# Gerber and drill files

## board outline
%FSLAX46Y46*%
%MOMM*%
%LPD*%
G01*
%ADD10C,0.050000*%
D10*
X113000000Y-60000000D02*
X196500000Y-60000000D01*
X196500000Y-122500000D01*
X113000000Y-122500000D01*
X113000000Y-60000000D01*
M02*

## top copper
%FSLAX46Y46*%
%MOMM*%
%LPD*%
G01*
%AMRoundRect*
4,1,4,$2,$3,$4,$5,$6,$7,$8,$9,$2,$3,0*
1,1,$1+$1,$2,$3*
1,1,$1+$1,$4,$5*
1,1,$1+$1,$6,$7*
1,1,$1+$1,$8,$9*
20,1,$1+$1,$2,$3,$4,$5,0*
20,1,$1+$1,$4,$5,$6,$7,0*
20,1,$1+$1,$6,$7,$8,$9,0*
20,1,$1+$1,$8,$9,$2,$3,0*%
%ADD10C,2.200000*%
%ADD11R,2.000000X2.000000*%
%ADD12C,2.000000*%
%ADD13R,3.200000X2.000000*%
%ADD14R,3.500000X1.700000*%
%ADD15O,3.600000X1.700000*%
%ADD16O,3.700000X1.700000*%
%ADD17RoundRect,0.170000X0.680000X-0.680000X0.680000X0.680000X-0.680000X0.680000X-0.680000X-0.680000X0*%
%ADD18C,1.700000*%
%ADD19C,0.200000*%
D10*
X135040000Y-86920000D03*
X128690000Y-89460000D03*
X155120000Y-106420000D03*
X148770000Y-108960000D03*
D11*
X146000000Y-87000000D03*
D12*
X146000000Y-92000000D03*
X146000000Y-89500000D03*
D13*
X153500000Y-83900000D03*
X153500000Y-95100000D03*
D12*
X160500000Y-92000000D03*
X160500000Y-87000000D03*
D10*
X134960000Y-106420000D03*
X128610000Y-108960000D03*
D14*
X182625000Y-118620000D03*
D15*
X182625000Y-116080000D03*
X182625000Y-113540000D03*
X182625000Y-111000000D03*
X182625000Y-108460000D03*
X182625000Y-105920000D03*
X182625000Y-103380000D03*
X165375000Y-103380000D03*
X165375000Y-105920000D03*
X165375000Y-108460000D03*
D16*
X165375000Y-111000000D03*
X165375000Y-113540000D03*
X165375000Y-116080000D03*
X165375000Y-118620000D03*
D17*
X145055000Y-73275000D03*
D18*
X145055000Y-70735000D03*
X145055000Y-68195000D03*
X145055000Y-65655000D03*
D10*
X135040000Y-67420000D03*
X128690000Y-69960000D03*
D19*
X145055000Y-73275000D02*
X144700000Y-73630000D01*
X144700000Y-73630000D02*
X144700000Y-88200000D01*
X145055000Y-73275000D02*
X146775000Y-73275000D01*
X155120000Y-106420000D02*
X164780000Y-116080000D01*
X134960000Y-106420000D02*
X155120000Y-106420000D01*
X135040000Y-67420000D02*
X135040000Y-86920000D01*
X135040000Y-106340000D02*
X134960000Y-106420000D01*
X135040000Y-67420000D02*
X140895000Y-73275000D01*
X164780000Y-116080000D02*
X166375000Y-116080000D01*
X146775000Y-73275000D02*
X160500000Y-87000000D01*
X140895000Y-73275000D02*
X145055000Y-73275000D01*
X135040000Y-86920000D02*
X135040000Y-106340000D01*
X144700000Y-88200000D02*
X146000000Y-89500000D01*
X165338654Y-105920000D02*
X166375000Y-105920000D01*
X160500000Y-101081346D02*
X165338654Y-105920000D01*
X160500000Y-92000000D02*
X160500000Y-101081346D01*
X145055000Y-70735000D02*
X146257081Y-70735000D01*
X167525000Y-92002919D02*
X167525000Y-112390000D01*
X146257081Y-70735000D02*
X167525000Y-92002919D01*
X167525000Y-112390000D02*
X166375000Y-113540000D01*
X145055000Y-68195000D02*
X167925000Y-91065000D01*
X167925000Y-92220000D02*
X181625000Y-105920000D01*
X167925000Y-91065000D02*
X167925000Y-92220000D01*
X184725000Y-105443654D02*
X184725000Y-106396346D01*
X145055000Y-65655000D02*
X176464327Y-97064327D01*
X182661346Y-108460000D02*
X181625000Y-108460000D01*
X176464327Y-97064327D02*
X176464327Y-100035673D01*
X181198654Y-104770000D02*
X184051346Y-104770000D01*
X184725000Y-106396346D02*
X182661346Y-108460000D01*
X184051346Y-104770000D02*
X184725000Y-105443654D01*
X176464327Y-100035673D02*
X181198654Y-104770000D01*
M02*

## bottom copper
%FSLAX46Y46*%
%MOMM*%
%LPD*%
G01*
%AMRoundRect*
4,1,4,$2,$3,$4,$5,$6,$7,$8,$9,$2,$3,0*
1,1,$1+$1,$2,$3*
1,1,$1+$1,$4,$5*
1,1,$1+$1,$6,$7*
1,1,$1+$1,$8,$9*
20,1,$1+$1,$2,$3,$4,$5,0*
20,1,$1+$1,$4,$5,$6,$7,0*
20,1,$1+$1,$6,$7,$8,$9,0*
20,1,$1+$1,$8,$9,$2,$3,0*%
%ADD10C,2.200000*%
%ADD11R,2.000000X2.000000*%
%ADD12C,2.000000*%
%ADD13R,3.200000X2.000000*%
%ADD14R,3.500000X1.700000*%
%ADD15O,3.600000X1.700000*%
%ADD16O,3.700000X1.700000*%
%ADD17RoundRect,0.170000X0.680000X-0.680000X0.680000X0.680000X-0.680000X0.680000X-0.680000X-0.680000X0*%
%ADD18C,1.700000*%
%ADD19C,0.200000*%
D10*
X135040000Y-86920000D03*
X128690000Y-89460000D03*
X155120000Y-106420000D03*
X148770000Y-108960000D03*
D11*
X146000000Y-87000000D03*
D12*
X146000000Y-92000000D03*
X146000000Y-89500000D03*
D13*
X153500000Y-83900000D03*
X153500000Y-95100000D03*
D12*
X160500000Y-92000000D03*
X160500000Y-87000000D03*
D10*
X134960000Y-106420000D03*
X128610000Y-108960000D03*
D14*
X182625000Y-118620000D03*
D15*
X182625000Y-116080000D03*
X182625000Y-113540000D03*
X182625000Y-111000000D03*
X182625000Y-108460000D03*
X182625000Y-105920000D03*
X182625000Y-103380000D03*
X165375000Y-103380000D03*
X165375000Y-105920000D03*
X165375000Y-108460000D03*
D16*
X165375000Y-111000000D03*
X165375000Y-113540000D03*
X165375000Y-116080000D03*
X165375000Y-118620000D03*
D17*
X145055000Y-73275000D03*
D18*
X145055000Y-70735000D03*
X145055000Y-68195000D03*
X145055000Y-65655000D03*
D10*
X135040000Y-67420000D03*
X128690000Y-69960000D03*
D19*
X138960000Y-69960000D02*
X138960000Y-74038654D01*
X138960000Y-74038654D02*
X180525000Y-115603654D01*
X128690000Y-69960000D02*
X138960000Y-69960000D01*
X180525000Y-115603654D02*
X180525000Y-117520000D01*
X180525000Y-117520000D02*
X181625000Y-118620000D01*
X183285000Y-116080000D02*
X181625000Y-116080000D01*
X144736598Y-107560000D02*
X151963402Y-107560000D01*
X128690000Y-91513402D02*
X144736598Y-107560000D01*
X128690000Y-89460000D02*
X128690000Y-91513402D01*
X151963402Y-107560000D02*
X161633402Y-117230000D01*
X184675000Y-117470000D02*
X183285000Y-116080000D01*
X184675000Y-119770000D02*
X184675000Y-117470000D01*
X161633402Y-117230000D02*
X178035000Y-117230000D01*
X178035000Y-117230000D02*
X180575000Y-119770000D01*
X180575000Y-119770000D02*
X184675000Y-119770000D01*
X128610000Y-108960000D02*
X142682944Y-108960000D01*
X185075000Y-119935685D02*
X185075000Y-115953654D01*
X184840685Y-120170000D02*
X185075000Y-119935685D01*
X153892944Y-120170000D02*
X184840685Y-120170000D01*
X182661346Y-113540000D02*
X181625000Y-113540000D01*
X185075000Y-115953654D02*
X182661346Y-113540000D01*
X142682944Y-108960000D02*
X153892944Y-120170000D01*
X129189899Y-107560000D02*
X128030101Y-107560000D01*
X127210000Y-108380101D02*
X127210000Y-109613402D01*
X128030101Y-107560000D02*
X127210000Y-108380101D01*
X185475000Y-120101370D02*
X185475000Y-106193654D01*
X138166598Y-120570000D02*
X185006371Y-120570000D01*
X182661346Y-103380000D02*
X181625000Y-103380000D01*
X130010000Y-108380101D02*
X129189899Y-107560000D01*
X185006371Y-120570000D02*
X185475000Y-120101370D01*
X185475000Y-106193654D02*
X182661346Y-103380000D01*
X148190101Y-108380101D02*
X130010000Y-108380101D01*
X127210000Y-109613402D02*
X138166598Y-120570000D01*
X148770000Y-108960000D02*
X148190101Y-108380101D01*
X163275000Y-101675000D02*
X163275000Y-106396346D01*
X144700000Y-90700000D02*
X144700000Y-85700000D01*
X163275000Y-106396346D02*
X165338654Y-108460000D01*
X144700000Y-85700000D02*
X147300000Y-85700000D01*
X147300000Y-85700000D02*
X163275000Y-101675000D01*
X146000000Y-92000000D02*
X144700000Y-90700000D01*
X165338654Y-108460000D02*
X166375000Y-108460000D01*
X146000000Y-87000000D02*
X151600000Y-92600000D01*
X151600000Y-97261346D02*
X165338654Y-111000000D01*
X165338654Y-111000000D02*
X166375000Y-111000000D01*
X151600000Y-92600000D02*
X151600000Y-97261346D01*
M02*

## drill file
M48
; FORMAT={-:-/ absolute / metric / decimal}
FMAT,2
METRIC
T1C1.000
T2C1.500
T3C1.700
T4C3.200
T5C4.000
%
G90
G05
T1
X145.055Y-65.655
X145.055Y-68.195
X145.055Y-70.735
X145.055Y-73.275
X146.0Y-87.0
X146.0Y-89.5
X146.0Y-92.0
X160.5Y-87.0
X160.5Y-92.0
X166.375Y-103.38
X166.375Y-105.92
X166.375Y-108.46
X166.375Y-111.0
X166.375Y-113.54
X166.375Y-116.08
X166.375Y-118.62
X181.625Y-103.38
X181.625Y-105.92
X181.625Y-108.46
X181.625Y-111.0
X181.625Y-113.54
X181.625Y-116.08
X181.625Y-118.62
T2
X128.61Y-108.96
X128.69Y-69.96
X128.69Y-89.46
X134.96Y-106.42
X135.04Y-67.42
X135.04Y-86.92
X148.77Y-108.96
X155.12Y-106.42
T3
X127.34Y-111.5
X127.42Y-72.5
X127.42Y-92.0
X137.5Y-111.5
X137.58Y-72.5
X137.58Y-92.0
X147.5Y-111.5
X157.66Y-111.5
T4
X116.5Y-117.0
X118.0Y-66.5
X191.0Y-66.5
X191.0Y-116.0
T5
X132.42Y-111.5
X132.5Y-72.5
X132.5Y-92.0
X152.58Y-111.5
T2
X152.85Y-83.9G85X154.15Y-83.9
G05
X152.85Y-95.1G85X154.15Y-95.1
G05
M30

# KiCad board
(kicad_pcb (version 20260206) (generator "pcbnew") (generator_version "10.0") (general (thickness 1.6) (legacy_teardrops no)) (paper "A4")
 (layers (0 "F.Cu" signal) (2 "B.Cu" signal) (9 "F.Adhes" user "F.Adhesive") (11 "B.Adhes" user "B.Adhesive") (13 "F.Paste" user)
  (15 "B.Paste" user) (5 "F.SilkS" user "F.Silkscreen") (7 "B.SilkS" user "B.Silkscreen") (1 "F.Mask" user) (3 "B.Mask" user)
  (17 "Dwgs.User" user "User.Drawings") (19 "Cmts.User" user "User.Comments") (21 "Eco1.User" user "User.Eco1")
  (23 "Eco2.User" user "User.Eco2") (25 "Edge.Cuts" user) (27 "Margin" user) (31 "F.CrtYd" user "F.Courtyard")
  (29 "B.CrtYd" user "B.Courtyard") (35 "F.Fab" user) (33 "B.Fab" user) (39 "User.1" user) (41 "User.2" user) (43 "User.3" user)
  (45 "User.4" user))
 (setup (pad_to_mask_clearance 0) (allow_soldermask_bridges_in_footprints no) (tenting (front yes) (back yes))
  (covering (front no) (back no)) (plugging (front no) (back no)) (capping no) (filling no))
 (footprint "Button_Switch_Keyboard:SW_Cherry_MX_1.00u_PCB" (layer "F.Cu") (at 135.04 86.92)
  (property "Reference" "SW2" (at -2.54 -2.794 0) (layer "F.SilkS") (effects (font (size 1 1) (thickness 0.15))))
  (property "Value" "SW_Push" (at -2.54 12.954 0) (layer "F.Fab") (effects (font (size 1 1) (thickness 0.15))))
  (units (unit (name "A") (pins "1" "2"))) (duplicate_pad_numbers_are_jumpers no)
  (pad "" np_thru_hole circle (at -7.62 5.08) (size 1.7 1.7) (drill 1.7) (layers "*.Cu" "*.Mask"))
  (pad "" np_thru_hole circle (at -2.54 5.08) (size 4 4) (drill 4) (layers "*.Cu" "*.Mask"))
  (pad "" np_thru_hole circle (at 2.54 5.08) (size 1.7 1.7) (drill 1.7) (layers "*.Cu" "*.Mask"))
  (pad "1" thru_hole circle (at 0 0) (size 2.2 2.2) (drill 1.5) (layers "*.Cu" "*.Mask") (remove_unused_layers no) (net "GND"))
  (pad "2" thru_hole circle (at -6.35 2.54) (size 2.2 2.2) (drill 1.5) (layers "*.Cu" "*.Mask") (remove_unused_layers no)
   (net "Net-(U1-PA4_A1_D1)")))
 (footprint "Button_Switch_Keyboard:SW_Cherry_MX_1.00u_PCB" (layer "F.Cu") (at 155.12 106.42)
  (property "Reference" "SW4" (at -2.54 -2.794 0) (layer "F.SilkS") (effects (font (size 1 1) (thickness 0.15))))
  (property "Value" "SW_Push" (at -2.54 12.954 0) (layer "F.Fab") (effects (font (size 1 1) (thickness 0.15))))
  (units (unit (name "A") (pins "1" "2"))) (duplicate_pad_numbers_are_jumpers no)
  (pad "" np_thru_hole circle (at -7.62 5.08) (size 1.7 1.7) (drill 1.7) (layers "*.Cu" "*.Mask"))
  (pad "" np_thru_hole circle (at -2.54 5.08) (size 4 4) (drill 4) (layers "*.Cu" "*.Mask"))
  (pad "" np_thru_hole circle (at 2.54 5.08) (size 1.7 1.7) (drill 1.7) (layers "*.Cu" "*.Mask"))
  (pad "1" thru_hole circle (at 0 0) (size 2.2 2.2) (drill 1.5) (layers "*.Cu" "*.Mask") (remove_unused_layers no) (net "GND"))
  (pad "2" thru_hole circle (at -6.35 2.54) (size 2.2 2.2) (drill 1.5) (layers "*.Cu" "*.Mask") (remove_unused_layers no)
   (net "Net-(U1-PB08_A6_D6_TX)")))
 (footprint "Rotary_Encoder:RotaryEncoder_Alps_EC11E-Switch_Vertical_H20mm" (layer "F.Cu") (at 146 87)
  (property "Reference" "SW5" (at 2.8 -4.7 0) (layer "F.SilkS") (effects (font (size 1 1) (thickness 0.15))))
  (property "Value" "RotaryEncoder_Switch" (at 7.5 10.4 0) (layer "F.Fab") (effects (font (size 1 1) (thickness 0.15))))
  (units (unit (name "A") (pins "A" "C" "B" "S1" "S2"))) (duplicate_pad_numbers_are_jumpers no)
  (pad "A" thru_hole rect (at 0 0) (size 2 2) (drill 1) (layers "*.Cu" "*.Mask") (remove_unused_layers no) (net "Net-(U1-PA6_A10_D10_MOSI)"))
  (pad "B" thru_hole circle (at 0 5) (size 2 2) (drill 1) (layers "*.Cu" "*.Mask") (remove_unused_layers no) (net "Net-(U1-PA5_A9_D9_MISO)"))
  (pad "C" thru_hole circle (at 0 2.5) (size 2 2) (drill 1) (layers "*.Cu" "*.Mask") (remove_unused_layers no) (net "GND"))
  (pad "MP" thru_hole rect (at 7.5 -3.1) (size 3.2 2) (drill oval 2.8 1.5) (layers "*.Cu" "*.Mask") (remove_unused_layers no))
  (pad "MP" thru_hole rect (at 7.5 8.1) (size 3.2 2) (drill oval 2.8 1.5) (layers "*.Cu" "*.Mask") (remove_unused_layers no))
  (pad "S1" thru_hole circle (at 14.5 5) (size 2 2) (drill 1) (layers "*.Cu" "*.Mask") (remove_unused_layers no)
   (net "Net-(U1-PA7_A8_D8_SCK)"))
  (pad "S2" thru_hole circle (at 14.5 0) (size 2 2) (drill 1) (layers "*.Cu" "*.Mask") (remove_unused_layers no) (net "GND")))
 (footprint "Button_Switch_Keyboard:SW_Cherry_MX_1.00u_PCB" (layer "F.Cu") (at 134.96 106.42)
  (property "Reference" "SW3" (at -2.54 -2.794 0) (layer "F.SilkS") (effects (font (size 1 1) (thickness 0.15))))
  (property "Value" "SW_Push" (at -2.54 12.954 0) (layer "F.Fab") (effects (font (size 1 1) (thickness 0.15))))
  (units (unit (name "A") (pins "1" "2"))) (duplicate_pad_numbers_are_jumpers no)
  (pad "" np_thru_hole circle (at -7.62 5.08) (size 1.7 1.7) (drill 1.7) (layers "*.Cu" "*.Mask"))
  (pad "" np_thru_hole circle (at -2.54 5.08) (size 4 4) (drill 4) (layers "*.Cu" "*.Mask"))
  (pad "" np_thru_hole circle (at 2.54 5.08) (size 1.7 1.7) (drill 1.7) (layers "*.Cu" "*.Mask"))
  (pad "1" thru_hole circle (at 0 0) (size 2.2 2.2) (drill 1.5) (layers "*.Cu" "*.Mask") (remove_unused_layers no) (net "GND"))
  (pad "2" thru_hole circle (at -6.35 2.54) (size 2.2 2.2) (drill 1.5) (layers "*.Cu" "*.Mask") (remove_unused_layers no)
   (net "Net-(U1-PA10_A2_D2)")))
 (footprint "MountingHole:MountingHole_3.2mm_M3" (layer "F.Cu") (at 116.5 117)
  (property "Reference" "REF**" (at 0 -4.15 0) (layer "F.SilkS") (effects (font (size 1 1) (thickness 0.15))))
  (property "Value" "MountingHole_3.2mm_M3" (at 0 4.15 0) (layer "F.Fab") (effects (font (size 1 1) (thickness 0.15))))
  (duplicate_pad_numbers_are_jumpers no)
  (pad "" np_thru_hole circle (at 0 0) (size 3.2 3.2) (drill 3.2) (layers "*.Cu" "*.Mask")))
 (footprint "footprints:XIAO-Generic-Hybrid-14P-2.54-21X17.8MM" (layer "F.Cu") (at 174 111 180)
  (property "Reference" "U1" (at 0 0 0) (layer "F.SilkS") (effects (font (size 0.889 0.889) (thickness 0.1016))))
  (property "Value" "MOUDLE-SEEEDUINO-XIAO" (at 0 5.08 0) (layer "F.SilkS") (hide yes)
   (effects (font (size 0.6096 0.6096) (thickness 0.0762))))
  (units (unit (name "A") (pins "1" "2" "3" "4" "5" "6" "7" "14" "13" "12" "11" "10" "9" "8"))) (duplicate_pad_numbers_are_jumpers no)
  (pad "1" thru_hole rect (at -7.625 -7.62 180) (size 3.5 1.7) (drill 1 (offset -1 0)) (layers "*.Cu" "*.Mask") (remove_unused_layers no)
   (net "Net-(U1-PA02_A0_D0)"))
  (pad "2" thru_hole oval (at -7.625 -5.08 180) (size 3.6 1.7) (drill 1 (offset -1 0)) (layers "*.Cu" "*.Mask") (remove_unused_layers no)
   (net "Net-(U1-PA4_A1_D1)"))
  (pad "3" thru_hole oval (at -7.625 -2.54 180) (size 3.6 1.7) (drill 1 (offset -1 0)) (layers "*.Cu" "*.Mask") (remove_unused_layers no)
   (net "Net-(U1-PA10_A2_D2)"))
  (pad "4" thru_hole oval (at -7.625 0 180) (size 3.6 1.7) (drill 1 (offset -1 0)) (layers "*.Cu" "*.Mask") (remove_unused_layers no)
   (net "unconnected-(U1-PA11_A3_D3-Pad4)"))
  (pad "5" thru_hole oval (at -7.625 2.54 180) (size 3.6 1.7) (drill 1 (offset -1 0)) (layers "*.Cu" "*.Mask") (remove_unused_layers no)
   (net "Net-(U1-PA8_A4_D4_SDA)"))
  (pad "6" thru_hole oval (at -7.625 5.08) (size 3.6 1.7) (drill 1 (offset 1 0)) (layers "*.Cu" "*.Mask") (remove_unused_layers no)
   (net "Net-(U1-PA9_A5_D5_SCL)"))
  (pad "7" thru_hole oval (at -7.625 7.62 180) (size 3.6 1.7) (drill 1 (offset -1 0)) (layers "*.Cu" "*.Mask") (remove_unused_layers no)
   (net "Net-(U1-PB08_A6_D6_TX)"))
  (pad "8" thru_hole oval (at 7.625 7.62 180) (size 3.6 1.7) (drill 1 (offset 1 0)) (layers "*.Cu" "*.Mask") (remove_unused_layers no)
   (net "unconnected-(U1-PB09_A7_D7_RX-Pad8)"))
  (pad "9" thru_hole oval (at 7.625 5.08 180) (size 3.6 1.7) (drill 1 (offset 1 0)) (layers "*.Cu" "*.Mask") (remove_unused_layers no)
   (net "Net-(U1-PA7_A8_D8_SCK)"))
  (pad "10" thru_hole oval (at 7.625 2.54 180) (size 3.6 1.7) (drill 1 (offset 1 0)) (layers "*.Cu" "*.Mask") (remove_unused_layers no)
   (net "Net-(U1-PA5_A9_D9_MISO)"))
  (pad "11" thru_hole oval (at 7.625 0 180) (size 3.7 1.7) (drill 1 (offset 1 0)) (layers "*.Cu" "*.Mask") (remove_unused_layers no)
   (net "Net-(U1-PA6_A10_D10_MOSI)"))
  (pad "12" thru_hole oval (at 7.625 -2.54 180) (size 3.7 1.7) (drill 1 (offset 1 0)) (layers "*.Cu" "*.Mask") (remove_unused_layers no)
   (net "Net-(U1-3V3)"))
  (pad "13" thru_hole oval (at 7.625 -5.08 180) (size 3.7 1.7) (drill 1 (offset 1 0)) (layers "*.Cu" "*.Mask") (remove_unused_layers no)
   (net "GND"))
  (pad "14" thru_hole oval (at 7.625 -7.62 180) (size 3.7 1.7) (drill 1 (offset 1 0)) (layers "*.Cu" "*.Mask") (remove_unused_layers no)
   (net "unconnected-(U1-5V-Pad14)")))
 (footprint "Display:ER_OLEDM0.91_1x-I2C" (layer "F.Cu") (at 145.055 73.275 90)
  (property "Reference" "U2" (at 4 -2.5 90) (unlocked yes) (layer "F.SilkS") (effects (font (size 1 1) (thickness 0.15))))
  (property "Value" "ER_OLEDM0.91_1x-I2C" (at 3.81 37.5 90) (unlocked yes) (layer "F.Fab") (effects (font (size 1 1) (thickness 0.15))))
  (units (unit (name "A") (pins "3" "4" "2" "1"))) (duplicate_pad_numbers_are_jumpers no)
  (pad "1" thru_hole roundrect (at 0 0 90) (size 1.7 1.7) (drill 1) (layers "*.Cu" "*.Mask") (remove_unused_layers no)
   (roundrect_rratio 0.1) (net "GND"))
  (pad "2" thru_hole circle (at 2.54 0 90) (size 1.7 1.7) (drill 1) (layers "*.Cu" "*.Mask") (remove_unused_layers no) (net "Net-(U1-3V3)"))
  (pad "3" thru_hole circle (at 5.08 0 90) (size 1.7 1.7) (drill 1) (layers "*.Cu" "*.Mask") (remove_unused_layers no)
   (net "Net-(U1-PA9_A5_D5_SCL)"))
  (pad "4" thru_hole circle (at 7.62 0 90) (size 1.7 1.7) (drill 1) (layers "*.Cu" "*.Mask") (remove_unused_layers no)
   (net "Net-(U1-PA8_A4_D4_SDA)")))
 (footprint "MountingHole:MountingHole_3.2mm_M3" (layer "F.Cu") (at 191 116)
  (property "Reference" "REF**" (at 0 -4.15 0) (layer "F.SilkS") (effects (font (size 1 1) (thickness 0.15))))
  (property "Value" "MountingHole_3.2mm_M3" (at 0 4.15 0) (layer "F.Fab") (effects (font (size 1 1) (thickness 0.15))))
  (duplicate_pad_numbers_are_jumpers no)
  (pad "" np_thru_hole circle (at 0 0) (size 3.2 3.2) (drill 3.2) (layers "*.Cu" "*.Mask")))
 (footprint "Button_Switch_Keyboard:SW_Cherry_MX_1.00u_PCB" (layer "F.Cu") (at 135.04 67.42)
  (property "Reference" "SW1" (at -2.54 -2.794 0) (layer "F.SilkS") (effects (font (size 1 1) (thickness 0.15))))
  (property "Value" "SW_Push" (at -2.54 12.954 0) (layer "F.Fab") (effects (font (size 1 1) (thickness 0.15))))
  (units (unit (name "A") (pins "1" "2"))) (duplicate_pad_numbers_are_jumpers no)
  (pad "" np_thru_hole circle (at -7.62 5.08) (size 1.7 1.7) (drill 1.7) (layers "*.Cu" "*.Mask"))
  (pad "" np_thru_hole circle (at -2.54 5.08) (size 4 4) (drill 4) (layers "*.Cu" "*.Mask"))
  (pad "" np_thru_hole circle (at 2.54 5.08) (size 1.7 1.7) (drill 1.7) (layers "*.Cu" "*.Mask"))
  (pad "1" thru_hole circle (at 0 0) (size 2.2 2.2) (drill 1.5) (layers "*.Cu" "*.Mask") (remove_unused_layers no) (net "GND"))
  (pad "2" thru_hole circle (at -6.35 2.54) (size 2.2 2.2) (drill 1.5) (layers "*.Cu" "*.Mask") (remove_unused_layers no)
   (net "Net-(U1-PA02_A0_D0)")))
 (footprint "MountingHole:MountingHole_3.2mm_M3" (layer "F.Cu") (at 118 66.5)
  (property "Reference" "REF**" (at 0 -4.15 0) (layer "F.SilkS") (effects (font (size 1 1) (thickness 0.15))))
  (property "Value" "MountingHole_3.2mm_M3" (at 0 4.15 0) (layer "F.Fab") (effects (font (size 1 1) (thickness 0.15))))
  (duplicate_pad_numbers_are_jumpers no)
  (pad "" np_thru_hole circle (at 0 0) (size 3.2 3.2) (drill 3.2) (layers "*.Cu" "*.Mask")))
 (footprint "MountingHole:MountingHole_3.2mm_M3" (layer "F.Cu") (at 191 66.5)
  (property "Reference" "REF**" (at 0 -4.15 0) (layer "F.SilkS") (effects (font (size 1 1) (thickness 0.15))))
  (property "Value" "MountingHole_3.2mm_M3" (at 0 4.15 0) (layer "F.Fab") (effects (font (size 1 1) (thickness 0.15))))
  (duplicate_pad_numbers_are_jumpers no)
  (pad "" np_thru_hole circle (at 0 0) (size 3.2 3.2) (drill 3.2) (layers "*.Cu" "*.Mask")))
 (gr_rect (start 113 60) (end 196.5 122.5) (stroke (width 0.05) (type default)) (fill no) (layer "Edge.Cuts"))
 (segment (start 145.055 73.275) (end 144.7 73.63) (width 0.2) (layer "F.Cu") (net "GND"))
 (segment (start 144.7 73.63) (end 144.7 88.2) (width 0.2) (layer "F.Cu") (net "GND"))
 (segment (start 145.055 73.275) (end 146.775 73.275) (width 0.2) (layer "F.Cu") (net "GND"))
 (segment (start 155.12 106.42) (end 164.78 116.08) (width 0.2) (layer "F.Cu") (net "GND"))
 (segment (start 134.96 106.42) (end 155.12 106.42) (width 0.2) (layer "F.Cu") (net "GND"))
 (segment (start 135.04 67.42) (end 135.04 86.92) (width 0.2) (layer "F.Cu") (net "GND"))
 (segment (start 135.04 106.34) (end 134.96 106.42) (width 0.2) (layer "F.Cu") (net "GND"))
 (segment (start 135.04 67.42) (end 140.895 73.275) (width 0.2) (layer "F.Cu") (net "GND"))
 (segment (start 164.78 116.08) (end 166.375 116.08) (width 0.2) (layer "F.Cu") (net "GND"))
 (segment (start 146.775 73.275) (end 160.5 87) (width 0.2) (layer "F.Cu") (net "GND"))
 (segment (start 140.895 73.275) (end 145.055 73.275) (width 0.2) (layer "F.Cu") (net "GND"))
 (segment (start 135.04 86.92) (end 135.04 106.34) (width 0.2) (layer "F.Cu") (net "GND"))
 (segment (start 144.7 88.2) (end 146 89.5) (width 0.2) (layer "F.Cu") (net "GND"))
 (segment (start 138.96 69.96) (end 138.96 74.038654) (width 0.2) (layer "B.Cu") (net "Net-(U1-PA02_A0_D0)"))
 (segment (start 138.96 74.038654) (end 180.525 115.603654) (width 0.2) (layer "B.Cu") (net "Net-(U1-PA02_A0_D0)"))
 (segment (start 128.69 69.96) (end 138.96 69.96) (width 0.2) (layer "B.Cu") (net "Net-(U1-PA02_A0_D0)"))
 (segment (start 180.525 115.603654) (end 180.525 117.52) (width 0.2) (layer "B.Cu") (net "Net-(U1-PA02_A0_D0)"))
 (segment (start 180.525 117.52) (end 181.625 118.62) (width 0.2) (layer "B.Cu") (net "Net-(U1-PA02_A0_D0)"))
 (segment (start 183.285 116.08) (end 181.625 116.08) (width 0.2) (layer "B.Cu") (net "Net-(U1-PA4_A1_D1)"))
 (segment (start 144.736598 107.56) (end 151.963402 107.56) (width 0.2) (layer "B.Cu") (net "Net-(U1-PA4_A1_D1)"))
 (segment (start 128.69 91.513402) (end 144.736598 107.56) (width 0.2) (layer "B.Cu") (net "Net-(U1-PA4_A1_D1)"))
 (segment (start 128.69 89.46) (end 128.69 91.513402) (width 0.2) (layer "B.Cu") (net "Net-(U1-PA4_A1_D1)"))
 (segment (start 151.963402 107.56) (end 161.633402 117.23) (width 0.2) (layer "B.Cu") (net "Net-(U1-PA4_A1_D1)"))
 (segment (start 184.675 117.47) (end 183.285 116.08) (width 0.2) (layer "B.Cu") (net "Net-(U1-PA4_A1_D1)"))
 (segment (start 184.675 119.77) (end 184.675 117.47) (width 0.2) (layer "B.Cu") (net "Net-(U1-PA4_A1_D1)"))
 (segment (start 161.633402 117.23) (end 178.035 117.23) (width 0.2) (layer "B.Cu") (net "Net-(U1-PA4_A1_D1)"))
 (segment (start 178.035 117.23) (end 180.575 119.77) (width 0.2) (layer "B.Cu") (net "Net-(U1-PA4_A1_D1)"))
 (segment (start 180.575 119.77) (end 184.675 119.77) (width 0.2) (layer "B.Cu") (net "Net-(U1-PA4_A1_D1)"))
 (segment (start 128.61 108.96) (end 142.682944 108.96) (width 0.2) (layer "B.Cu") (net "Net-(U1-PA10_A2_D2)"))
 (segment (start 185.075 119.935685) (end 185.075 115.953654) (width 0.2) (layer "B.Cu") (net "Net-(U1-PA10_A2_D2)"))
 (segment (start 184.840685 120.17) (end 185.075 119.935685) (width 0.2) (layer "B.Cu") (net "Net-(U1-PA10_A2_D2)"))
 (segment (start 153.892944 120.17) (end 184.840685 120.17) (width 0.2) (layer "B.Cu") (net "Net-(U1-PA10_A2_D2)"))
 (segment (start 182.661346 113.54) (end 181.625 113.54) (width 0.2) (layer "B.Cu") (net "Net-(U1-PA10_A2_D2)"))
 (segment (start 185.075 115.953654) (end 182.661346 113.54) (width 0.2) (layer "B.Cu") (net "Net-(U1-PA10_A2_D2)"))
 (segment (start 142.682944 108.96) (end 153.892944 120.17) (width 0.2) (layer "B.Cu") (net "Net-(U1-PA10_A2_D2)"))
 (segment (start 129.189899 107.56) (end 128.030101 107.56) (width 0.2) (layer "B.Cu") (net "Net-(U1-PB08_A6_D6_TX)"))
 (segment (start 127.21 108.380101) (end 127.21 109.613402) (width 0.2) (layer "B.Cu") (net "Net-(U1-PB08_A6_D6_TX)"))
 (segment (start 128.030101 107.56) (end 127.21 108.380101) (width 0.2) (layer "B.Cu") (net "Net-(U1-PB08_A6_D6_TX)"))
 (segment (start 185.475 120.10137) (end 185.475 106.193654) (width 0.2) (layer "B.Cu") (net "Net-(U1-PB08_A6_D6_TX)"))
 (segment (start 138.166598 120.57) (end 185.006371 120.57) (width 0.2) (layer "B.Cu") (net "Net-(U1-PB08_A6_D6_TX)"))
 (segment (start 182.661346 103.38) (end 181.625 103.38) (width 0.2) (layer "B.Cu") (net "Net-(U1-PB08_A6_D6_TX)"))
 (segment (start 130.01 108.380101) (end 129.189899 107.56) (width 0.2) (layer "B.Cu") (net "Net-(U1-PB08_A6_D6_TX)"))
 (segment (start 185.006371 120.57) (end 185.475 120.10137) (width 0.2) (layer "B.Cu") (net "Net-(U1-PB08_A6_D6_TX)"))
 (segment (start 185.475 106.193654) (end 182.661346 103.38) (width 0.2) (layer "B.Cu") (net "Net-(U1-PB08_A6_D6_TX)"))
 (segment (start 148.190101 108.380101) (end 130.01 108.380101) (width 0.2) (layer "B.Cu") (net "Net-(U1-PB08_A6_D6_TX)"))
 (segment (start 127.21 109.613402) (end 138.166598 120.57) (width 0.2) (layer "B.Cu") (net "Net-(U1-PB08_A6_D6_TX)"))
 (segment (start 148.77 108.96) (end 148.190101 108.380101) (width 0.2) (layer "B.Cu") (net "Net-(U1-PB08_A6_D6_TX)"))
 (segment (start 165.338654 105.92) (end 166.375 105.92) (width 0.2) (layer "F.Cu") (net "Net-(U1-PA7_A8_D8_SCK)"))
 (segment (start 160.5 101.081346) (end 165.338654 105.92) (width 0.2) (layer "F.Cu") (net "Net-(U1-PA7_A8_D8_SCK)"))
 (segment (start 160.5 92) (end 160.5 101.081346) (width 0.2) (layer "F.Cu") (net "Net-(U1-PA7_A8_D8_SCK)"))
 (segment (start 163.275 101.675) (end 163.275 106.396346) (width 0.2) (layer "B.Cu") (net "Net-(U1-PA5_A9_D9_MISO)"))
 (segment (start 144.7 90.7) (end 144.7 85.7) (width 0.2) (layer "B.Cu") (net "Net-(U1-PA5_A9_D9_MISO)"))
 (segment (start 163.275 106.396346) (end 165.338654 108.46) (width 0.2) (layer "B.Cu") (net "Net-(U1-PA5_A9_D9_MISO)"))
 (segment (start 144.7 85.7) (end 147.3 85.7) (width 0.2) (layer "B.Cu") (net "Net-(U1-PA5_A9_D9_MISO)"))
 (segment (start 147.3 85.7) (end 163.275 101.675) (width 0.2) (layer "B.Cu") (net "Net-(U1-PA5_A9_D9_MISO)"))
 (segment (start 146 92) (end 144.7 90.7) (width 0.2) (layer "B.Cu") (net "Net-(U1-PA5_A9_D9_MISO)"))
 (segment (start 165.338654 108.46) (end 166.375 108.46) (width 0.2) (layer "B.Cu") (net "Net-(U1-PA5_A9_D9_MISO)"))
 (segment (start 146 87) (end 151.6 92.6) (width 0.2) (layer "B.Cu") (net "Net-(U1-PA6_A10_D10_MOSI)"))
 (segment (start 151.6 97.261346) (end 165.338654 111) (width 0.2) (layer "B.Cu") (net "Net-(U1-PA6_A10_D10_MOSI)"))
 (segment (start 165.338654 111) (end 166.375 111) (width 0.2) (layer "B.Cu") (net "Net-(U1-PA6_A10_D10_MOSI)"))
 (segment (start 151.6 92.6) (end 151.6 97.261346) (width 0.2) (layer "B.Cu") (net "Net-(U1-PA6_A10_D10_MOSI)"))
 (segment (start 145.055 70.735) (end 146.257081 70.735) (width 0.2) (layer "F.Cu") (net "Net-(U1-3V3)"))
 (segment (start 167.525 92.002919) (end 167.525 112.39) (width 0.2) (layer "F.Cu") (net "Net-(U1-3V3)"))
 (segment (start 146.257081 70.735) (end 167.525 92.002919) (width 0.2) (layer "F.Cu") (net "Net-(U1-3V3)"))
 (segment (start 167.525 112.39) (end 166.375 113.54) (width 0.2) (layer "F.Cu") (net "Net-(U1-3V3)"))
 (segment (start 145.055 68.195) (end 167.925 91.065) (width 0.2) (layer "F.Cu") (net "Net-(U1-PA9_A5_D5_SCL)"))
 (segment (start 167.925 92.22) (end 181.625 105.92) (width 0.2) (layer "F.Cu") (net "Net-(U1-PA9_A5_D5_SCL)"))
 (segment (start 167.925 91.065) (end 167.925 92.22) (width 0.2) (layer "F.Cu") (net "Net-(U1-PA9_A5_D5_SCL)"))
 (segment (start 184.725 105.443654) (end 184.725 106.396346) (width 0.2) (layer "F.Cu") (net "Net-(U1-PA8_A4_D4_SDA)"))
 (segment (start 145.055 65.655) (end 176.464327 97.064327) (width 0.2) (layer "F.Cu") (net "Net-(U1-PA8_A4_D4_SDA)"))
 (segment (start 182.661346 108.46) (end 181.625 108.46) (width 0.2) (layer "F.Cu") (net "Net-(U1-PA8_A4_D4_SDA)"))
 (segment (start 176.464327 97.064327) (end 176.464327 100.035673) (width 0.2) (layer "F.Cu") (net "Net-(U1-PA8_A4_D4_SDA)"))
 (segment (start 181.198654 104.77) (end 184.051346 104.77) (width 0.2) (layer "F.Cu") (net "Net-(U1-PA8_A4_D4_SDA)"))
 (segment (start 184.725 106.396346) (end 182.661346 108.46) (width 0.2) (layer "F.Cu") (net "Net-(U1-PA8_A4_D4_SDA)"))
 (segment (start 184.051346 104.77) (end 184.725 105.443654) (width 0.2) (layer "F.Cu") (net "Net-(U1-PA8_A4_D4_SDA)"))
 (segment (start 176.464327 100.035673) (end 181.198654 104.77) (width 0.2) (layer "F.Cu") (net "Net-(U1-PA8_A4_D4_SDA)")))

